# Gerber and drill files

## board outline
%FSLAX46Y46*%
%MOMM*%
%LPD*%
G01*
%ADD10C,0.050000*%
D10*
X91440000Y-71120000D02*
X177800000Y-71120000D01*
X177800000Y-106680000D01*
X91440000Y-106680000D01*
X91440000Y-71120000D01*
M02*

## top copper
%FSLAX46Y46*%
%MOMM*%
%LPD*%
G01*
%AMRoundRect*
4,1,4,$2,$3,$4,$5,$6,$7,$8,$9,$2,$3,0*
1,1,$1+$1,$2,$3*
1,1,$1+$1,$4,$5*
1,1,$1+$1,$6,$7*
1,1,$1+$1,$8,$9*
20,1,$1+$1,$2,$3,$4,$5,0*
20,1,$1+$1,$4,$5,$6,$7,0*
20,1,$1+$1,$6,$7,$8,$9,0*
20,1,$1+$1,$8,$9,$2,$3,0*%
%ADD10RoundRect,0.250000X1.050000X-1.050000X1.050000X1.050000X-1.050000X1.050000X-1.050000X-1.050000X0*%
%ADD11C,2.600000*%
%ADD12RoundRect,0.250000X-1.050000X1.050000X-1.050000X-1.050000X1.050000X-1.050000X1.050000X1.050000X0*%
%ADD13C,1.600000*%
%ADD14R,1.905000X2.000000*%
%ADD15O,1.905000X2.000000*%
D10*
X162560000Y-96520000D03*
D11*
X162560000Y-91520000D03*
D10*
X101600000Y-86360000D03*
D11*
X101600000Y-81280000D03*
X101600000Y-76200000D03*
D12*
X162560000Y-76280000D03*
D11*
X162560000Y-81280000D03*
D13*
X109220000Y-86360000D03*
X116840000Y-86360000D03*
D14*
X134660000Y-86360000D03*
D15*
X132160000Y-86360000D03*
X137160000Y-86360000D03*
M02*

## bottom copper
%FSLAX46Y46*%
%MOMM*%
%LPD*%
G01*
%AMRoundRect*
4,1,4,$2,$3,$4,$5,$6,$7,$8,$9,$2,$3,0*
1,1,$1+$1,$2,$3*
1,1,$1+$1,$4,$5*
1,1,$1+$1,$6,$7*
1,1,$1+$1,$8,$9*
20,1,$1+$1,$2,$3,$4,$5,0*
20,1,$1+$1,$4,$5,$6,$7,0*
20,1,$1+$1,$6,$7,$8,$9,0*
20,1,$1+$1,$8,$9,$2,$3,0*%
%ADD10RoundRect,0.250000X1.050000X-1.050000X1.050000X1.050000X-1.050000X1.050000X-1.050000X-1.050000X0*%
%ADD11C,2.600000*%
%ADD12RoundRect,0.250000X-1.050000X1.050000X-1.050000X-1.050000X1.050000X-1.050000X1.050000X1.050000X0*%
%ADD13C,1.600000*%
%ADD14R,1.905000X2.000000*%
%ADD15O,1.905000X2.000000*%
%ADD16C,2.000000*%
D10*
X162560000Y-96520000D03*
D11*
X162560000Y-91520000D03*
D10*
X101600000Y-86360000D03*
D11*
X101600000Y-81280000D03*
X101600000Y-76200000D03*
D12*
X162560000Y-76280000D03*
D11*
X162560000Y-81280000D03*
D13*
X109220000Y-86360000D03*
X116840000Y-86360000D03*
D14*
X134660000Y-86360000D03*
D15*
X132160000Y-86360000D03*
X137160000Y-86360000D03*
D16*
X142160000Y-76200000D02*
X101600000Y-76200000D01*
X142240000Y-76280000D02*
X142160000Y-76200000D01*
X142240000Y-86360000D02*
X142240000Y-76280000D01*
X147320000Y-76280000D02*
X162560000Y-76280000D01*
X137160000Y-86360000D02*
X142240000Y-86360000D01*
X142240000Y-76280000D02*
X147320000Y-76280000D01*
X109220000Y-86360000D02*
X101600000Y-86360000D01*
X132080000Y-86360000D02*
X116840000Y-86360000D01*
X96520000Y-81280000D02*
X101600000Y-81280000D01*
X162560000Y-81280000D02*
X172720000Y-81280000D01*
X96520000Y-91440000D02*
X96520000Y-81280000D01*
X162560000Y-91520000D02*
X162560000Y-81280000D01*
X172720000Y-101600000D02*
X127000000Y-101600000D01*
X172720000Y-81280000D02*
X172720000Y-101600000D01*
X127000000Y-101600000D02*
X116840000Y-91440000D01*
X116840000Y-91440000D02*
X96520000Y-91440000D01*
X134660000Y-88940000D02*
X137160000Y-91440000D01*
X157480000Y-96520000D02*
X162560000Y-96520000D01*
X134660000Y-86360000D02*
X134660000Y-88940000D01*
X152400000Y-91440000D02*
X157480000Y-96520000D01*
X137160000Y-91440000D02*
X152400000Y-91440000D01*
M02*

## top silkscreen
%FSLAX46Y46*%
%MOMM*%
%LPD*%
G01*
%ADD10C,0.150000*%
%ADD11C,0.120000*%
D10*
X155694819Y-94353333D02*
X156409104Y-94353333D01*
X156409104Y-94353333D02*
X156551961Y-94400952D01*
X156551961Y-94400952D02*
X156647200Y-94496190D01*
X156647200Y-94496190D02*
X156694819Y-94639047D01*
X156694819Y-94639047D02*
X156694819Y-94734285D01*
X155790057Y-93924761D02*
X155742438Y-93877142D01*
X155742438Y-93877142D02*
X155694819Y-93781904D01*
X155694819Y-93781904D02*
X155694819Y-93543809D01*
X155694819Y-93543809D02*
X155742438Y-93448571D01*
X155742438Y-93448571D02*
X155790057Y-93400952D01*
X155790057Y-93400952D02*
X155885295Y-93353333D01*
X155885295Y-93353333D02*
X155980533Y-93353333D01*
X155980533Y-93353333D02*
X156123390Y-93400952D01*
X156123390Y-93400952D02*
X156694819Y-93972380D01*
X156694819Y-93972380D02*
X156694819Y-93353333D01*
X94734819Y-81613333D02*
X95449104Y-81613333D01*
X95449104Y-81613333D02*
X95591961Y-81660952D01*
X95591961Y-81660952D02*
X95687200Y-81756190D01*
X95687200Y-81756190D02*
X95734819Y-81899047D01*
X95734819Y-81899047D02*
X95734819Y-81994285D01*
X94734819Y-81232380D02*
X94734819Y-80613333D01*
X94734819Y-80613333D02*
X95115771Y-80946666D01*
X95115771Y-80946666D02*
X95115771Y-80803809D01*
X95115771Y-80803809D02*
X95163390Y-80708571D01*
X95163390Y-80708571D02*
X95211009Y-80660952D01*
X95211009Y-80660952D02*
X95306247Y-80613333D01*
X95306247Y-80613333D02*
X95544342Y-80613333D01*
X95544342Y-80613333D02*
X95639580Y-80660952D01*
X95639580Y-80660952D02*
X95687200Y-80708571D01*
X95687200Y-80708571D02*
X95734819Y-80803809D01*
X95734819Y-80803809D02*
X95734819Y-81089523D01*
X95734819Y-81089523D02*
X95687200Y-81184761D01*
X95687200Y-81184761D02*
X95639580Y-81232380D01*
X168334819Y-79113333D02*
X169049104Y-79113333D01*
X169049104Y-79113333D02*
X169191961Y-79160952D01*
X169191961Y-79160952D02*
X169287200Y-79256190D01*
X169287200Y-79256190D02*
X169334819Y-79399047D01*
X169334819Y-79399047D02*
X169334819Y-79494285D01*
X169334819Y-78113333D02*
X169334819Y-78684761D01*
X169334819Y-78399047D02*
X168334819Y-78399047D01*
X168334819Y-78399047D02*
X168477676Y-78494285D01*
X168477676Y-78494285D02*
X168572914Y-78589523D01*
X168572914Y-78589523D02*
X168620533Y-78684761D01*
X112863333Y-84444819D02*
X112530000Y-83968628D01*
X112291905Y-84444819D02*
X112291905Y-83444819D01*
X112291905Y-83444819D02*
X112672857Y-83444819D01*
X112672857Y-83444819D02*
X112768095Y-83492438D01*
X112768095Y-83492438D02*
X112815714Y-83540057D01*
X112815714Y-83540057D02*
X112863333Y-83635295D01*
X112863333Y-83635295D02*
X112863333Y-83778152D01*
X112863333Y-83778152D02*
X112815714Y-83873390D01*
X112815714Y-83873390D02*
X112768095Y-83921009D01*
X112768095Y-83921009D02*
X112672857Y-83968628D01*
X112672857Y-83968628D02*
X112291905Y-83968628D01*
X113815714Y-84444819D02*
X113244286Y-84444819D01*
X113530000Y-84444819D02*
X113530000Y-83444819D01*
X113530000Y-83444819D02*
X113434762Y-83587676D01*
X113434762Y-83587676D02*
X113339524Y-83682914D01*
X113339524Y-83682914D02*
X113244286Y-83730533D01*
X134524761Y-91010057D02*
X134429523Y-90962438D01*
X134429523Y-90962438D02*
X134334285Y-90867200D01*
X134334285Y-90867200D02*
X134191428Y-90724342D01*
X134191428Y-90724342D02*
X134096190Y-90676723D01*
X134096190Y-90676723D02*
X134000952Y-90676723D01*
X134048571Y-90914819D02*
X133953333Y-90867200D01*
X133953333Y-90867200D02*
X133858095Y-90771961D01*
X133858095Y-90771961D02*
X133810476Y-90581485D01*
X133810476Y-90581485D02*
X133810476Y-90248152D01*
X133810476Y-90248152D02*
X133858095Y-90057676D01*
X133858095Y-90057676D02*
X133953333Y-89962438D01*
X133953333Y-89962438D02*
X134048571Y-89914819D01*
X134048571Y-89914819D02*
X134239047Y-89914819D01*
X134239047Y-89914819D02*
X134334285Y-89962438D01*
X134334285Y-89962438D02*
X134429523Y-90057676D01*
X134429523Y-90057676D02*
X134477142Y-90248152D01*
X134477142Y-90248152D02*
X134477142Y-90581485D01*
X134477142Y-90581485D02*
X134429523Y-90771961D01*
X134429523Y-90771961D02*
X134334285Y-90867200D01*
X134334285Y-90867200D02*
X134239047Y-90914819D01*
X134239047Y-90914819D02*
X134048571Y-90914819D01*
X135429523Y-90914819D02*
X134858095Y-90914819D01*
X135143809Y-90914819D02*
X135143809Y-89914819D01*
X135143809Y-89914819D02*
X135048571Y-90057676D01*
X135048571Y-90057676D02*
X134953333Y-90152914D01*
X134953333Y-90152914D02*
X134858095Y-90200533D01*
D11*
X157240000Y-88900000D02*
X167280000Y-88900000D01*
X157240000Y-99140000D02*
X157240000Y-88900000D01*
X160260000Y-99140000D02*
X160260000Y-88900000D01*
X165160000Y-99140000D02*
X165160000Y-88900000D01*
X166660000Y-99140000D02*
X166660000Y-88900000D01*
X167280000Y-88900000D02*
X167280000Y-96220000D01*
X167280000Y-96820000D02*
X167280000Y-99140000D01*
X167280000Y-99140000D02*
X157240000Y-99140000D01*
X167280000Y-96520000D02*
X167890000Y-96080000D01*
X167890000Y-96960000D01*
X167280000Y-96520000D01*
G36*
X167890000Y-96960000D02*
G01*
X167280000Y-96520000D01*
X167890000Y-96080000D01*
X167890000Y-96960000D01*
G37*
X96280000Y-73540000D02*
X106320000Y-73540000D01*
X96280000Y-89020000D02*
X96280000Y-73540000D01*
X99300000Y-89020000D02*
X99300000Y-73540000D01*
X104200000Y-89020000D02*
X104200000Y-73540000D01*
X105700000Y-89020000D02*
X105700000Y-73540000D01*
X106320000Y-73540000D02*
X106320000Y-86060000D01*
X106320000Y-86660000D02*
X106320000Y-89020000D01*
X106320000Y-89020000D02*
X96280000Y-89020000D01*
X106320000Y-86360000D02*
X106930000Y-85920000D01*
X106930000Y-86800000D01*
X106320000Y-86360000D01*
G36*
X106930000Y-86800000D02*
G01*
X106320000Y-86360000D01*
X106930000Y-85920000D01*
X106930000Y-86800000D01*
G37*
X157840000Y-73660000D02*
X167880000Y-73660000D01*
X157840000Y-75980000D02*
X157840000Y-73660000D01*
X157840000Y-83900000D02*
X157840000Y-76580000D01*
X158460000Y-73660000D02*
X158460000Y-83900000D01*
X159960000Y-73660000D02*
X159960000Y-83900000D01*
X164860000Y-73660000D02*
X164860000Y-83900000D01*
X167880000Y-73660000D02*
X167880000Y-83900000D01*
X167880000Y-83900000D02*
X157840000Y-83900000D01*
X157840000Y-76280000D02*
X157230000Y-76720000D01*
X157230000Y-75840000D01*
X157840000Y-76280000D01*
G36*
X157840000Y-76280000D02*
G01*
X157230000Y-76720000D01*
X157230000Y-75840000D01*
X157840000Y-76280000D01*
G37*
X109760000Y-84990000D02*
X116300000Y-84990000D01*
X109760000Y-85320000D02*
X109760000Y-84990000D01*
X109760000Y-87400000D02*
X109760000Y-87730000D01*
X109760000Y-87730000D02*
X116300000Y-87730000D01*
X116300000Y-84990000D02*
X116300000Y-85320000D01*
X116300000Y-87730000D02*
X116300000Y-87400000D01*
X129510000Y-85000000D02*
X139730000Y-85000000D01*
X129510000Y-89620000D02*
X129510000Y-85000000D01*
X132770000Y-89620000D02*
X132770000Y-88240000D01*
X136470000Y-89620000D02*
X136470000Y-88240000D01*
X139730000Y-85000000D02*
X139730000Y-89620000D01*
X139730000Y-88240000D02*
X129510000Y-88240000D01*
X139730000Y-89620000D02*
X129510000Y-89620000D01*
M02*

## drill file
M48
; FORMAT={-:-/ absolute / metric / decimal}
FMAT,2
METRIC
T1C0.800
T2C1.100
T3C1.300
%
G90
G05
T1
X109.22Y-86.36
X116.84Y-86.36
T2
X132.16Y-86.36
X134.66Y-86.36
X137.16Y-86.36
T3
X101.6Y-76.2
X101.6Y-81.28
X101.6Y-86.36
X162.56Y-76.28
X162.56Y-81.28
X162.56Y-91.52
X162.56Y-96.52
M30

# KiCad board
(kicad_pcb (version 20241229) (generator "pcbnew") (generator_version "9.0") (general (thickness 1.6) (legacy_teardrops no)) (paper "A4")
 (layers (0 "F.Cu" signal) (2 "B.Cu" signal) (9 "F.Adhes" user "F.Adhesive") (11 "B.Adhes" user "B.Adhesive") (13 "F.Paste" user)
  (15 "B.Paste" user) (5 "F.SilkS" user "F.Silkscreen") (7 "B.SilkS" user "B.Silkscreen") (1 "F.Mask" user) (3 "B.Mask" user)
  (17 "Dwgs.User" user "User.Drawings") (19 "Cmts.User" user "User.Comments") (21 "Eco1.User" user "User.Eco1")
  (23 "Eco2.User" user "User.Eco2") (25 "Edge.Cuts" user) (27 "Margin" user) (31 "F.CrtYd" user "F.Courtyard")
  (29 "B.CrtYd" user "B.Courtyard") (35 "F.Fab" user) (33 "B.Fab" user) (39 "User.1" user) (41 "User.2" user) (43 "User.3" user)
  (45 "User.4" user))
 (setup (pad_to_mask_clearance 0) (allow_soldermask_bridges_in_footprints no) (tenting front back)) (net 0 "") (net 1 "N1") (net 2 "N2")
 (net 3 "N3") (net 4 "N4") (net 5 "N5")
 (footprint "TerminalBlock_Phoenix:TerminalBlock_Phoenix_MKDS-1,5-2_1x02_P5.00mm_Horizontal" (layer "F.Cu") (at 162.56 96.52 90)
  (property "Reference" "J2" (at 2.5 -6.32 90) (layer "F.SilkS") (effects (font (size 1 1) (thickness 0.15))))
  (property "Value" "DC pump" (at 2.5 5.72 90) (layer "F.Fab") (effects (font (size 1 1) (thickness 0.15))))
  (fp_line (start 7.62 -5.32) (end 7.62 4.72) (stroke (width 0.12) (type solid)) (layer "F.SilkS"))
  (fp_line (start -2.62 -5.32) (end 7.62 -5.32) (stroke (width 0.12) (type solid)) (layer "F.SilkS"))
  (fp_line (start -2.62 -2.3) (end 7.62 -2.3) (stroke (width 0.12) (type solid)) (layer "F.SilkS"))
  (fp_line (start -2.62 2.6) (end 7.62 2.6) (stroke (width 0.12) (type solid)) (layer "F.SilkS"))
  (fp_line (start -2.62 4.1) (end 7.62 4.1) (stroke (width 0.12) (type solid)) (layer "F.SilkS"))
  (fp_line (start 7.62 4.72) (end 0.3 4.72) (stroke (width 0.12) (type solid)) (layer "F.SilkS"))
  (fp_line (start -0.3 4.72) (end -2.62 4.72) (stroke (width 0.12) (type solid)) (layer "F.SilkS"))
  (fp_line (start -2.62 4.72) (end -2.62 -5.32) (stroke (width 0.12) (type solid)) (layer "F.SilkS"))
  (fp_poly (pts (xy 0 4.72) (xy 0.44 5.33) (xy -0.44 5.33)) (stroke (width 0.12) (type solid)) (fill yes) (layer "F.SilkS"))
  (pad "1" thru_hole roundrect (at 0 0 90) (size 2.6 2.6) (drill 1.3) (layers "*.Cu" "*.Mask") (remove_unused_layers no)
   (roundrect_rratio 0.096154) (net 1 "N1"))
  (pad "2" thru_hole circle (at 5 0 90) (size 2.6 2.6) (drill 1.3) (layers "*.Cu" "*.Mask") (remove_unused_layers no) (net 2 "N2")))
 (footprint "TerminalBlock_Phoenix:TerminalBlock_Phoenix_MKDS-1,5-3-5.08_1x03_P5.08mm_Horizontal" (layer "F.Cu") (at 101.6 86.36 90)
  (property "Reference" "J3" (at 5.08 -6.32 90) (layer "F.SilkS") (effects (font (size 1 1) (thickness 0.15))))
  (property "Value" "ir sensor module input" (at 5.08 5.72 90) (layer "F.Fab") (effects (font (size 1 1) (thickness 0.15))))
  (fp_line (start 12.82 -5.32) (end 12.82 4.72) (stroke (width 0.12) (type solid)) (layer "F.SilkS"))
  (fp_line (start -2.66 -5.32) (end 12.82 -5.32) (stroke (width 0.12) (type solid)) (layer "F.SilkS"))
  (fp_line (start -2.66 -2.3) (end 12.82 -2.3) (stroke (width 0.12) (type solid)) (layer "F.SilkS"))
  (fp_line (start -2.66 2.6) (end 12.82 2.6) (stroke (width 0.12) (type solid)) (layer "F.SilkS"))
  (fp_line (start -2.66 4.1) (end 12.82 4.1) (stroke (width 0.12) (type solid)) (layer "F.SilkS"))
  (fp_line (start 12.82 4.72) (end 0.3 4.72) (stroke (width 0.12) (type solid)) (layer "F.SilkS"))
  (fp_line (start -0.3 4.72) (end -2.66 4.72) (stroke (width 0.12) (type solid)) (layer "F.SilkS"))
  (fp_line (start -2.66 4.72) (end -2.66 -5.32) (stroke (width 0.12) (type solid)) (layer "F.SilkS"))
  (fp_poly (pts (xy 0 4.72) (xy 0.44 5.33) (xy -0.44 5.33)) (stroke (width 0.12) (type solid)) (fill yes) (layer "F.SilkS"))
  (pad "1" thru_hole roundrect (at 0 0 90) (size 2.6 2.6) (drill 1.3) (layers "*.Cu" "*.Mask") (remove_unused_layers no)
   (roundrect_rratio 0.096154) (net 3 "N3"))
  (pad "2" thru_hole circle (at 5.08 0 90) (size 2.6 2.6) (drill 1.3) (layers "*.Cu" "*.Mask") (remove_unused_layers no) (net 2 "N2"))
  (pad "3" thru_hole circle (at 10.16 0 90) (size 2.6 2.6) (drill 1.3) (layers "*.Cu" "*.Mask") (remove_unused_layers no) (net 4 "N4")))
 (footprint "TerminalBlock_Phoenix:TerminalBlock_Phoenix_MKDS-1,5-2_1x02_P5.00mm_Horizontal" (layer "F.Cu") (at 162.56 76.28 -90)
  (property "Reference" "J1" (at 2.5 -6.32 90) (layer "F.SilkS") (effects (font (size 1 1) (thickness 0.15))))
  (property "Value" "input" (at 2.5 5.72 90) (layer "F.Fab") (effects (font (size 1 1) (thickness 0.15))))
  (fp_line (start -2.62 4.72) (end -2.62 -5.32) (stroke (width 0.12) (type solid)) (layer "F.SilkS"))
  (fp_line (start -0.3 4.72) (end -2.62 4.72) (stroke (width 0.12) (type solid)) (layer "F.SilkS"))
  (fp_line (start 7.62 4.72) (end 0.3 4.72) (stroke (width 0.12) (type solid)) (layer "F.SilkS"))
  (fp_line (start -2.62 4.1) (end 7.62 4.1) (stroke (width 0.12) (type solid)) (layer "F.SilkS"))
  (fp_line (start -2.62 2.6) (end 7.62 2.6) (stroke (width 0.12) (type solid)) (layer "F.SilkS"))
  (fp_line (start -2.62 -2.3) (end 7.62 -2.3) (stroke (width 0.12) (type solid)) (layer "F.SilkS"))
  (fp_line (start -2.62 -5.32) (end 7.62 -5.32) (stroke (width 0.12) (type solid)) (layer "F.SilkS"))
  (fp_line (start 7.62 -5.32) (end 7.62 4.72) (stroke (width 0.12) (type solid)) (layer "F.SilkS"))
  (fp_poly (pts (xy 0 4.72) (xy 0.44 5.33) (xy -0.44 5.33)) (stroke (width 0.12) (type solid)) (fill yes) (layer "F.SilkS"))
  (pad "1" thru_hole roundrect (at 0 0 270) (size 2.6 2.6) (drill 1.3) (layers "*.Cu" "*.Mask") (remove_unused_layers no)
   (roundrect_rratio 0.096154) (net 4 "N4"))
  (pad "2" thru_hole circle (at 5 0 270) (size 2.6 2.6) (drill 1.3) (layers "*.Cu" "*.Mask") (remove_unused_layers no) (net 2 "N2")))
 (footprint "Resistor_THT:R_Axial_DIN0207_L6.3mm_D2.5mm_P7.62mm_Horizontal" (layer "F.Cu") (at 109.22 86.36)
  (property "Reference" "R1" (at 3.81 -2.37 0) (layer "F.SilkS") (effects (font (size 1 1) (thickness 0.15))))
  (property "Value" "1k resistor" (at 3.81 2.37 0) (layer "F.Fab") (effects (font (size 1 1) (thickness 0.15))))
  (fp_line (start 0.54 -1.37) (end 7.08 -1.37) (stroke (width 0.12) (type solid)) (layer "F.SilkS"))
  (fp_line (start 0.54 -1.04) (end 0.54 -1.37) (stroke (width 0.12) (type solid)) (layer "F.SilkS"))
  (fp_line (start 0.54 1.04) (end 0.54 1.37) (stroke (width 0.12) (type solid)) (layer "F.SilkS"))
  (fp_line (start 0.54 1.37) (end 7.08 1.37) (stroke (width 0.12) (type solid)) (layer "F.SilkS"))
  (fp_line (start 7.08 -1.37) (end 7.08 -1.04) (stroke (width 0.12) (type solid)) (layer "F.SilkS"))
  (fp_line (start 7.08 1.37) (end 7.08 1.04) (stroke (width 0.12) (type solid)) (layer "F.SilkS"))
  (pad "1" thru_hole circle (at 0 0) (size 1.6 1.6) (drill 0.8) (layers "*.Cu" "*.Mask") (remove_unused_layers no) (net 3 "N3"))
  (pad "2" thru_hole circle (at 7.62 0) (size 1.6 1.6) (drill 0.8) (layers "*.Cu" "*.Mask") (remove_unused_layers no) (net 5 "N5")))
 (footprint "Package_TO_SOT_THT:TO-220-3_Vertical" (layer "F.Cu") (at 137.16 86.36 180)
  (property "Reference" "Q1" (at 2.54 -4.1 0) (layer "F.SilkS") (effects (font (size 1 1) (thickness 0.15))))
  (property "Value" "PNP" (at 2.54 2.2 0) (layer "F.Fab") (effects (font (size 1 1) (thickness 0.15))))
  (fp_line (start 7.65 1.36) (end -2.57 1.36) (stroke (width 0.12) (type solid)) (layer "F.SilkS"))
  (fp_line (start 7.65 -3.26) (end 7.65 1.36) (stroke (width 0.12) (type solid)) (layer "F.SilkS"))
  (fp_line (start 4.39 -3.26) (end 4.39 -1.88) (stroke (width 0.12) (type solid)) (layer "F.SilkS"))
  (fp_line (start 0.69 -3.26) (end 0.69 -1.88) (stroke (width 0.12) (type solid)) (layer "F.SilkS"))
  (fp_line (start -2.57 1.36) (end -2.57 -3.26) (stroke (width 0.12) (type solid)) (layer "F.SilkS"))
  (fp_line (start -2.57 -1.88) (end 7.65 -1.88) (stroke (width 0.12) (type solid)) (layer "F.SilkS"))
  (fp_line (start -2.57 -3.26) (end 7.65 -3.26) (stroke (width 0.12) (type solid)) (layer "F.SilkS"))
  (pad "1" thru_hole rect (at 2.5 0 180) (size 1.905 2) (drill 1.1) (layers "*.Cu" "*.Mask") (remove_unused_layers no) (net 1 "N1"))
  (pad "2" thru_hole oval (at 5 0 180) (size 1.905 2) (drill 1.1) (layers "*.Cu" "*.Mask") (remove_unused_layers no) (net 5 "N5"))
  (pad "3" thru_hole oval (at 0 0 180) (size 1.905 2) (drill 1.1) (layers "*.Cu" "*.Mask") (remove_unused_layers no) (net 4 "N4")))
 (gr_rect (start 91.44 71.12) (end 177.8 106.68) (stroke (width 0.05) (type default)) (fill no) (layer "Edge.Cuts"))
 (segment (start 142.16 76.2) (end 101.6 76.2) (width 2) (layer "B.Cu") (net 4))
 (segment (start 142.24 76.28) (end 142.16 76.2) (width 2) (layer "B.Cu") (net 4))
 (segment (start 142.24 86.36) (end 142.24 76.28) (width 2) (layer "B.Cu") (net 4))
 (segment (start 147.32 76.28) (end 162.56 76.28) (width 2) (layer "B.Cu") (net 4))
 (segment (start 137.16 86.36) (end 142.24 86.36) (width 2) (layer "B.Cu") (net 4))
 (segment (start 142.24 76.28) (end 147.32 76.28) (width 2) (layer "B.Cu") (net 4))
 (segment (start 109.22 86.36) (end 101.6 86.36) (width 2) (layer "B.Cu") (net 3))
 (segment (start 132.08 86.36) (end 116.84 86.36) (width 2) (layer "B.Cu") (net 5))
 (segment (start 96.52 81.28) (end 101.6 81.28) (width 2) (layer "B.Cu") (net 2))
 (segment (start 162.56 81.28) (end 172.72 81.28) (width 2) (layer "B.Cu") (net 2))
 (segment (start 96.52 91.44) (end 96.52 81.28) (width 2) (layer "B.Cu") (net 2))
 (segment (start 162.56 91.52) (end 162.56 81.28) (width 2) (layer "B.Cu") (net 2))
 (segment (start 172.72 101.6) (end 127 101.6) (width 2) (layer "B.Cu") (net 2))
 (segment (start 172.72 81.28) (end 172.72 101.6) (width 2) (layer "B.Cu") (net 2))
 (segment (start 127 101.6) (end 116.84 91.44) (width 2) (layer "B.Cu") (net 2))
 (segment (start 116.84 91.44) (end 96.52 91.44) (width 2) (layer "B.Cu") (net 2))
 (segment (start 134.66 88.94) (end 137.16 91.44) (width 2) (layer "B.Cu") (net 1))
 (segment (start 157.48 96.52) (end 162.56 96.52) (width 2) (layer "B.Cu") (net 1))
 (segment (start 134.66 86.36) (end 134.66 88.94) (width 2) (layer "B.Cu") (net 1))
 (segment (start 152.4 91.44) (end 157.48 96.52) (width 2) (layer "B.Cu") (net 1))
 (segment (start 137.16 91.44) (end 152.4 91.44) (width 2) (layer "B.Cu") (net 1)))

